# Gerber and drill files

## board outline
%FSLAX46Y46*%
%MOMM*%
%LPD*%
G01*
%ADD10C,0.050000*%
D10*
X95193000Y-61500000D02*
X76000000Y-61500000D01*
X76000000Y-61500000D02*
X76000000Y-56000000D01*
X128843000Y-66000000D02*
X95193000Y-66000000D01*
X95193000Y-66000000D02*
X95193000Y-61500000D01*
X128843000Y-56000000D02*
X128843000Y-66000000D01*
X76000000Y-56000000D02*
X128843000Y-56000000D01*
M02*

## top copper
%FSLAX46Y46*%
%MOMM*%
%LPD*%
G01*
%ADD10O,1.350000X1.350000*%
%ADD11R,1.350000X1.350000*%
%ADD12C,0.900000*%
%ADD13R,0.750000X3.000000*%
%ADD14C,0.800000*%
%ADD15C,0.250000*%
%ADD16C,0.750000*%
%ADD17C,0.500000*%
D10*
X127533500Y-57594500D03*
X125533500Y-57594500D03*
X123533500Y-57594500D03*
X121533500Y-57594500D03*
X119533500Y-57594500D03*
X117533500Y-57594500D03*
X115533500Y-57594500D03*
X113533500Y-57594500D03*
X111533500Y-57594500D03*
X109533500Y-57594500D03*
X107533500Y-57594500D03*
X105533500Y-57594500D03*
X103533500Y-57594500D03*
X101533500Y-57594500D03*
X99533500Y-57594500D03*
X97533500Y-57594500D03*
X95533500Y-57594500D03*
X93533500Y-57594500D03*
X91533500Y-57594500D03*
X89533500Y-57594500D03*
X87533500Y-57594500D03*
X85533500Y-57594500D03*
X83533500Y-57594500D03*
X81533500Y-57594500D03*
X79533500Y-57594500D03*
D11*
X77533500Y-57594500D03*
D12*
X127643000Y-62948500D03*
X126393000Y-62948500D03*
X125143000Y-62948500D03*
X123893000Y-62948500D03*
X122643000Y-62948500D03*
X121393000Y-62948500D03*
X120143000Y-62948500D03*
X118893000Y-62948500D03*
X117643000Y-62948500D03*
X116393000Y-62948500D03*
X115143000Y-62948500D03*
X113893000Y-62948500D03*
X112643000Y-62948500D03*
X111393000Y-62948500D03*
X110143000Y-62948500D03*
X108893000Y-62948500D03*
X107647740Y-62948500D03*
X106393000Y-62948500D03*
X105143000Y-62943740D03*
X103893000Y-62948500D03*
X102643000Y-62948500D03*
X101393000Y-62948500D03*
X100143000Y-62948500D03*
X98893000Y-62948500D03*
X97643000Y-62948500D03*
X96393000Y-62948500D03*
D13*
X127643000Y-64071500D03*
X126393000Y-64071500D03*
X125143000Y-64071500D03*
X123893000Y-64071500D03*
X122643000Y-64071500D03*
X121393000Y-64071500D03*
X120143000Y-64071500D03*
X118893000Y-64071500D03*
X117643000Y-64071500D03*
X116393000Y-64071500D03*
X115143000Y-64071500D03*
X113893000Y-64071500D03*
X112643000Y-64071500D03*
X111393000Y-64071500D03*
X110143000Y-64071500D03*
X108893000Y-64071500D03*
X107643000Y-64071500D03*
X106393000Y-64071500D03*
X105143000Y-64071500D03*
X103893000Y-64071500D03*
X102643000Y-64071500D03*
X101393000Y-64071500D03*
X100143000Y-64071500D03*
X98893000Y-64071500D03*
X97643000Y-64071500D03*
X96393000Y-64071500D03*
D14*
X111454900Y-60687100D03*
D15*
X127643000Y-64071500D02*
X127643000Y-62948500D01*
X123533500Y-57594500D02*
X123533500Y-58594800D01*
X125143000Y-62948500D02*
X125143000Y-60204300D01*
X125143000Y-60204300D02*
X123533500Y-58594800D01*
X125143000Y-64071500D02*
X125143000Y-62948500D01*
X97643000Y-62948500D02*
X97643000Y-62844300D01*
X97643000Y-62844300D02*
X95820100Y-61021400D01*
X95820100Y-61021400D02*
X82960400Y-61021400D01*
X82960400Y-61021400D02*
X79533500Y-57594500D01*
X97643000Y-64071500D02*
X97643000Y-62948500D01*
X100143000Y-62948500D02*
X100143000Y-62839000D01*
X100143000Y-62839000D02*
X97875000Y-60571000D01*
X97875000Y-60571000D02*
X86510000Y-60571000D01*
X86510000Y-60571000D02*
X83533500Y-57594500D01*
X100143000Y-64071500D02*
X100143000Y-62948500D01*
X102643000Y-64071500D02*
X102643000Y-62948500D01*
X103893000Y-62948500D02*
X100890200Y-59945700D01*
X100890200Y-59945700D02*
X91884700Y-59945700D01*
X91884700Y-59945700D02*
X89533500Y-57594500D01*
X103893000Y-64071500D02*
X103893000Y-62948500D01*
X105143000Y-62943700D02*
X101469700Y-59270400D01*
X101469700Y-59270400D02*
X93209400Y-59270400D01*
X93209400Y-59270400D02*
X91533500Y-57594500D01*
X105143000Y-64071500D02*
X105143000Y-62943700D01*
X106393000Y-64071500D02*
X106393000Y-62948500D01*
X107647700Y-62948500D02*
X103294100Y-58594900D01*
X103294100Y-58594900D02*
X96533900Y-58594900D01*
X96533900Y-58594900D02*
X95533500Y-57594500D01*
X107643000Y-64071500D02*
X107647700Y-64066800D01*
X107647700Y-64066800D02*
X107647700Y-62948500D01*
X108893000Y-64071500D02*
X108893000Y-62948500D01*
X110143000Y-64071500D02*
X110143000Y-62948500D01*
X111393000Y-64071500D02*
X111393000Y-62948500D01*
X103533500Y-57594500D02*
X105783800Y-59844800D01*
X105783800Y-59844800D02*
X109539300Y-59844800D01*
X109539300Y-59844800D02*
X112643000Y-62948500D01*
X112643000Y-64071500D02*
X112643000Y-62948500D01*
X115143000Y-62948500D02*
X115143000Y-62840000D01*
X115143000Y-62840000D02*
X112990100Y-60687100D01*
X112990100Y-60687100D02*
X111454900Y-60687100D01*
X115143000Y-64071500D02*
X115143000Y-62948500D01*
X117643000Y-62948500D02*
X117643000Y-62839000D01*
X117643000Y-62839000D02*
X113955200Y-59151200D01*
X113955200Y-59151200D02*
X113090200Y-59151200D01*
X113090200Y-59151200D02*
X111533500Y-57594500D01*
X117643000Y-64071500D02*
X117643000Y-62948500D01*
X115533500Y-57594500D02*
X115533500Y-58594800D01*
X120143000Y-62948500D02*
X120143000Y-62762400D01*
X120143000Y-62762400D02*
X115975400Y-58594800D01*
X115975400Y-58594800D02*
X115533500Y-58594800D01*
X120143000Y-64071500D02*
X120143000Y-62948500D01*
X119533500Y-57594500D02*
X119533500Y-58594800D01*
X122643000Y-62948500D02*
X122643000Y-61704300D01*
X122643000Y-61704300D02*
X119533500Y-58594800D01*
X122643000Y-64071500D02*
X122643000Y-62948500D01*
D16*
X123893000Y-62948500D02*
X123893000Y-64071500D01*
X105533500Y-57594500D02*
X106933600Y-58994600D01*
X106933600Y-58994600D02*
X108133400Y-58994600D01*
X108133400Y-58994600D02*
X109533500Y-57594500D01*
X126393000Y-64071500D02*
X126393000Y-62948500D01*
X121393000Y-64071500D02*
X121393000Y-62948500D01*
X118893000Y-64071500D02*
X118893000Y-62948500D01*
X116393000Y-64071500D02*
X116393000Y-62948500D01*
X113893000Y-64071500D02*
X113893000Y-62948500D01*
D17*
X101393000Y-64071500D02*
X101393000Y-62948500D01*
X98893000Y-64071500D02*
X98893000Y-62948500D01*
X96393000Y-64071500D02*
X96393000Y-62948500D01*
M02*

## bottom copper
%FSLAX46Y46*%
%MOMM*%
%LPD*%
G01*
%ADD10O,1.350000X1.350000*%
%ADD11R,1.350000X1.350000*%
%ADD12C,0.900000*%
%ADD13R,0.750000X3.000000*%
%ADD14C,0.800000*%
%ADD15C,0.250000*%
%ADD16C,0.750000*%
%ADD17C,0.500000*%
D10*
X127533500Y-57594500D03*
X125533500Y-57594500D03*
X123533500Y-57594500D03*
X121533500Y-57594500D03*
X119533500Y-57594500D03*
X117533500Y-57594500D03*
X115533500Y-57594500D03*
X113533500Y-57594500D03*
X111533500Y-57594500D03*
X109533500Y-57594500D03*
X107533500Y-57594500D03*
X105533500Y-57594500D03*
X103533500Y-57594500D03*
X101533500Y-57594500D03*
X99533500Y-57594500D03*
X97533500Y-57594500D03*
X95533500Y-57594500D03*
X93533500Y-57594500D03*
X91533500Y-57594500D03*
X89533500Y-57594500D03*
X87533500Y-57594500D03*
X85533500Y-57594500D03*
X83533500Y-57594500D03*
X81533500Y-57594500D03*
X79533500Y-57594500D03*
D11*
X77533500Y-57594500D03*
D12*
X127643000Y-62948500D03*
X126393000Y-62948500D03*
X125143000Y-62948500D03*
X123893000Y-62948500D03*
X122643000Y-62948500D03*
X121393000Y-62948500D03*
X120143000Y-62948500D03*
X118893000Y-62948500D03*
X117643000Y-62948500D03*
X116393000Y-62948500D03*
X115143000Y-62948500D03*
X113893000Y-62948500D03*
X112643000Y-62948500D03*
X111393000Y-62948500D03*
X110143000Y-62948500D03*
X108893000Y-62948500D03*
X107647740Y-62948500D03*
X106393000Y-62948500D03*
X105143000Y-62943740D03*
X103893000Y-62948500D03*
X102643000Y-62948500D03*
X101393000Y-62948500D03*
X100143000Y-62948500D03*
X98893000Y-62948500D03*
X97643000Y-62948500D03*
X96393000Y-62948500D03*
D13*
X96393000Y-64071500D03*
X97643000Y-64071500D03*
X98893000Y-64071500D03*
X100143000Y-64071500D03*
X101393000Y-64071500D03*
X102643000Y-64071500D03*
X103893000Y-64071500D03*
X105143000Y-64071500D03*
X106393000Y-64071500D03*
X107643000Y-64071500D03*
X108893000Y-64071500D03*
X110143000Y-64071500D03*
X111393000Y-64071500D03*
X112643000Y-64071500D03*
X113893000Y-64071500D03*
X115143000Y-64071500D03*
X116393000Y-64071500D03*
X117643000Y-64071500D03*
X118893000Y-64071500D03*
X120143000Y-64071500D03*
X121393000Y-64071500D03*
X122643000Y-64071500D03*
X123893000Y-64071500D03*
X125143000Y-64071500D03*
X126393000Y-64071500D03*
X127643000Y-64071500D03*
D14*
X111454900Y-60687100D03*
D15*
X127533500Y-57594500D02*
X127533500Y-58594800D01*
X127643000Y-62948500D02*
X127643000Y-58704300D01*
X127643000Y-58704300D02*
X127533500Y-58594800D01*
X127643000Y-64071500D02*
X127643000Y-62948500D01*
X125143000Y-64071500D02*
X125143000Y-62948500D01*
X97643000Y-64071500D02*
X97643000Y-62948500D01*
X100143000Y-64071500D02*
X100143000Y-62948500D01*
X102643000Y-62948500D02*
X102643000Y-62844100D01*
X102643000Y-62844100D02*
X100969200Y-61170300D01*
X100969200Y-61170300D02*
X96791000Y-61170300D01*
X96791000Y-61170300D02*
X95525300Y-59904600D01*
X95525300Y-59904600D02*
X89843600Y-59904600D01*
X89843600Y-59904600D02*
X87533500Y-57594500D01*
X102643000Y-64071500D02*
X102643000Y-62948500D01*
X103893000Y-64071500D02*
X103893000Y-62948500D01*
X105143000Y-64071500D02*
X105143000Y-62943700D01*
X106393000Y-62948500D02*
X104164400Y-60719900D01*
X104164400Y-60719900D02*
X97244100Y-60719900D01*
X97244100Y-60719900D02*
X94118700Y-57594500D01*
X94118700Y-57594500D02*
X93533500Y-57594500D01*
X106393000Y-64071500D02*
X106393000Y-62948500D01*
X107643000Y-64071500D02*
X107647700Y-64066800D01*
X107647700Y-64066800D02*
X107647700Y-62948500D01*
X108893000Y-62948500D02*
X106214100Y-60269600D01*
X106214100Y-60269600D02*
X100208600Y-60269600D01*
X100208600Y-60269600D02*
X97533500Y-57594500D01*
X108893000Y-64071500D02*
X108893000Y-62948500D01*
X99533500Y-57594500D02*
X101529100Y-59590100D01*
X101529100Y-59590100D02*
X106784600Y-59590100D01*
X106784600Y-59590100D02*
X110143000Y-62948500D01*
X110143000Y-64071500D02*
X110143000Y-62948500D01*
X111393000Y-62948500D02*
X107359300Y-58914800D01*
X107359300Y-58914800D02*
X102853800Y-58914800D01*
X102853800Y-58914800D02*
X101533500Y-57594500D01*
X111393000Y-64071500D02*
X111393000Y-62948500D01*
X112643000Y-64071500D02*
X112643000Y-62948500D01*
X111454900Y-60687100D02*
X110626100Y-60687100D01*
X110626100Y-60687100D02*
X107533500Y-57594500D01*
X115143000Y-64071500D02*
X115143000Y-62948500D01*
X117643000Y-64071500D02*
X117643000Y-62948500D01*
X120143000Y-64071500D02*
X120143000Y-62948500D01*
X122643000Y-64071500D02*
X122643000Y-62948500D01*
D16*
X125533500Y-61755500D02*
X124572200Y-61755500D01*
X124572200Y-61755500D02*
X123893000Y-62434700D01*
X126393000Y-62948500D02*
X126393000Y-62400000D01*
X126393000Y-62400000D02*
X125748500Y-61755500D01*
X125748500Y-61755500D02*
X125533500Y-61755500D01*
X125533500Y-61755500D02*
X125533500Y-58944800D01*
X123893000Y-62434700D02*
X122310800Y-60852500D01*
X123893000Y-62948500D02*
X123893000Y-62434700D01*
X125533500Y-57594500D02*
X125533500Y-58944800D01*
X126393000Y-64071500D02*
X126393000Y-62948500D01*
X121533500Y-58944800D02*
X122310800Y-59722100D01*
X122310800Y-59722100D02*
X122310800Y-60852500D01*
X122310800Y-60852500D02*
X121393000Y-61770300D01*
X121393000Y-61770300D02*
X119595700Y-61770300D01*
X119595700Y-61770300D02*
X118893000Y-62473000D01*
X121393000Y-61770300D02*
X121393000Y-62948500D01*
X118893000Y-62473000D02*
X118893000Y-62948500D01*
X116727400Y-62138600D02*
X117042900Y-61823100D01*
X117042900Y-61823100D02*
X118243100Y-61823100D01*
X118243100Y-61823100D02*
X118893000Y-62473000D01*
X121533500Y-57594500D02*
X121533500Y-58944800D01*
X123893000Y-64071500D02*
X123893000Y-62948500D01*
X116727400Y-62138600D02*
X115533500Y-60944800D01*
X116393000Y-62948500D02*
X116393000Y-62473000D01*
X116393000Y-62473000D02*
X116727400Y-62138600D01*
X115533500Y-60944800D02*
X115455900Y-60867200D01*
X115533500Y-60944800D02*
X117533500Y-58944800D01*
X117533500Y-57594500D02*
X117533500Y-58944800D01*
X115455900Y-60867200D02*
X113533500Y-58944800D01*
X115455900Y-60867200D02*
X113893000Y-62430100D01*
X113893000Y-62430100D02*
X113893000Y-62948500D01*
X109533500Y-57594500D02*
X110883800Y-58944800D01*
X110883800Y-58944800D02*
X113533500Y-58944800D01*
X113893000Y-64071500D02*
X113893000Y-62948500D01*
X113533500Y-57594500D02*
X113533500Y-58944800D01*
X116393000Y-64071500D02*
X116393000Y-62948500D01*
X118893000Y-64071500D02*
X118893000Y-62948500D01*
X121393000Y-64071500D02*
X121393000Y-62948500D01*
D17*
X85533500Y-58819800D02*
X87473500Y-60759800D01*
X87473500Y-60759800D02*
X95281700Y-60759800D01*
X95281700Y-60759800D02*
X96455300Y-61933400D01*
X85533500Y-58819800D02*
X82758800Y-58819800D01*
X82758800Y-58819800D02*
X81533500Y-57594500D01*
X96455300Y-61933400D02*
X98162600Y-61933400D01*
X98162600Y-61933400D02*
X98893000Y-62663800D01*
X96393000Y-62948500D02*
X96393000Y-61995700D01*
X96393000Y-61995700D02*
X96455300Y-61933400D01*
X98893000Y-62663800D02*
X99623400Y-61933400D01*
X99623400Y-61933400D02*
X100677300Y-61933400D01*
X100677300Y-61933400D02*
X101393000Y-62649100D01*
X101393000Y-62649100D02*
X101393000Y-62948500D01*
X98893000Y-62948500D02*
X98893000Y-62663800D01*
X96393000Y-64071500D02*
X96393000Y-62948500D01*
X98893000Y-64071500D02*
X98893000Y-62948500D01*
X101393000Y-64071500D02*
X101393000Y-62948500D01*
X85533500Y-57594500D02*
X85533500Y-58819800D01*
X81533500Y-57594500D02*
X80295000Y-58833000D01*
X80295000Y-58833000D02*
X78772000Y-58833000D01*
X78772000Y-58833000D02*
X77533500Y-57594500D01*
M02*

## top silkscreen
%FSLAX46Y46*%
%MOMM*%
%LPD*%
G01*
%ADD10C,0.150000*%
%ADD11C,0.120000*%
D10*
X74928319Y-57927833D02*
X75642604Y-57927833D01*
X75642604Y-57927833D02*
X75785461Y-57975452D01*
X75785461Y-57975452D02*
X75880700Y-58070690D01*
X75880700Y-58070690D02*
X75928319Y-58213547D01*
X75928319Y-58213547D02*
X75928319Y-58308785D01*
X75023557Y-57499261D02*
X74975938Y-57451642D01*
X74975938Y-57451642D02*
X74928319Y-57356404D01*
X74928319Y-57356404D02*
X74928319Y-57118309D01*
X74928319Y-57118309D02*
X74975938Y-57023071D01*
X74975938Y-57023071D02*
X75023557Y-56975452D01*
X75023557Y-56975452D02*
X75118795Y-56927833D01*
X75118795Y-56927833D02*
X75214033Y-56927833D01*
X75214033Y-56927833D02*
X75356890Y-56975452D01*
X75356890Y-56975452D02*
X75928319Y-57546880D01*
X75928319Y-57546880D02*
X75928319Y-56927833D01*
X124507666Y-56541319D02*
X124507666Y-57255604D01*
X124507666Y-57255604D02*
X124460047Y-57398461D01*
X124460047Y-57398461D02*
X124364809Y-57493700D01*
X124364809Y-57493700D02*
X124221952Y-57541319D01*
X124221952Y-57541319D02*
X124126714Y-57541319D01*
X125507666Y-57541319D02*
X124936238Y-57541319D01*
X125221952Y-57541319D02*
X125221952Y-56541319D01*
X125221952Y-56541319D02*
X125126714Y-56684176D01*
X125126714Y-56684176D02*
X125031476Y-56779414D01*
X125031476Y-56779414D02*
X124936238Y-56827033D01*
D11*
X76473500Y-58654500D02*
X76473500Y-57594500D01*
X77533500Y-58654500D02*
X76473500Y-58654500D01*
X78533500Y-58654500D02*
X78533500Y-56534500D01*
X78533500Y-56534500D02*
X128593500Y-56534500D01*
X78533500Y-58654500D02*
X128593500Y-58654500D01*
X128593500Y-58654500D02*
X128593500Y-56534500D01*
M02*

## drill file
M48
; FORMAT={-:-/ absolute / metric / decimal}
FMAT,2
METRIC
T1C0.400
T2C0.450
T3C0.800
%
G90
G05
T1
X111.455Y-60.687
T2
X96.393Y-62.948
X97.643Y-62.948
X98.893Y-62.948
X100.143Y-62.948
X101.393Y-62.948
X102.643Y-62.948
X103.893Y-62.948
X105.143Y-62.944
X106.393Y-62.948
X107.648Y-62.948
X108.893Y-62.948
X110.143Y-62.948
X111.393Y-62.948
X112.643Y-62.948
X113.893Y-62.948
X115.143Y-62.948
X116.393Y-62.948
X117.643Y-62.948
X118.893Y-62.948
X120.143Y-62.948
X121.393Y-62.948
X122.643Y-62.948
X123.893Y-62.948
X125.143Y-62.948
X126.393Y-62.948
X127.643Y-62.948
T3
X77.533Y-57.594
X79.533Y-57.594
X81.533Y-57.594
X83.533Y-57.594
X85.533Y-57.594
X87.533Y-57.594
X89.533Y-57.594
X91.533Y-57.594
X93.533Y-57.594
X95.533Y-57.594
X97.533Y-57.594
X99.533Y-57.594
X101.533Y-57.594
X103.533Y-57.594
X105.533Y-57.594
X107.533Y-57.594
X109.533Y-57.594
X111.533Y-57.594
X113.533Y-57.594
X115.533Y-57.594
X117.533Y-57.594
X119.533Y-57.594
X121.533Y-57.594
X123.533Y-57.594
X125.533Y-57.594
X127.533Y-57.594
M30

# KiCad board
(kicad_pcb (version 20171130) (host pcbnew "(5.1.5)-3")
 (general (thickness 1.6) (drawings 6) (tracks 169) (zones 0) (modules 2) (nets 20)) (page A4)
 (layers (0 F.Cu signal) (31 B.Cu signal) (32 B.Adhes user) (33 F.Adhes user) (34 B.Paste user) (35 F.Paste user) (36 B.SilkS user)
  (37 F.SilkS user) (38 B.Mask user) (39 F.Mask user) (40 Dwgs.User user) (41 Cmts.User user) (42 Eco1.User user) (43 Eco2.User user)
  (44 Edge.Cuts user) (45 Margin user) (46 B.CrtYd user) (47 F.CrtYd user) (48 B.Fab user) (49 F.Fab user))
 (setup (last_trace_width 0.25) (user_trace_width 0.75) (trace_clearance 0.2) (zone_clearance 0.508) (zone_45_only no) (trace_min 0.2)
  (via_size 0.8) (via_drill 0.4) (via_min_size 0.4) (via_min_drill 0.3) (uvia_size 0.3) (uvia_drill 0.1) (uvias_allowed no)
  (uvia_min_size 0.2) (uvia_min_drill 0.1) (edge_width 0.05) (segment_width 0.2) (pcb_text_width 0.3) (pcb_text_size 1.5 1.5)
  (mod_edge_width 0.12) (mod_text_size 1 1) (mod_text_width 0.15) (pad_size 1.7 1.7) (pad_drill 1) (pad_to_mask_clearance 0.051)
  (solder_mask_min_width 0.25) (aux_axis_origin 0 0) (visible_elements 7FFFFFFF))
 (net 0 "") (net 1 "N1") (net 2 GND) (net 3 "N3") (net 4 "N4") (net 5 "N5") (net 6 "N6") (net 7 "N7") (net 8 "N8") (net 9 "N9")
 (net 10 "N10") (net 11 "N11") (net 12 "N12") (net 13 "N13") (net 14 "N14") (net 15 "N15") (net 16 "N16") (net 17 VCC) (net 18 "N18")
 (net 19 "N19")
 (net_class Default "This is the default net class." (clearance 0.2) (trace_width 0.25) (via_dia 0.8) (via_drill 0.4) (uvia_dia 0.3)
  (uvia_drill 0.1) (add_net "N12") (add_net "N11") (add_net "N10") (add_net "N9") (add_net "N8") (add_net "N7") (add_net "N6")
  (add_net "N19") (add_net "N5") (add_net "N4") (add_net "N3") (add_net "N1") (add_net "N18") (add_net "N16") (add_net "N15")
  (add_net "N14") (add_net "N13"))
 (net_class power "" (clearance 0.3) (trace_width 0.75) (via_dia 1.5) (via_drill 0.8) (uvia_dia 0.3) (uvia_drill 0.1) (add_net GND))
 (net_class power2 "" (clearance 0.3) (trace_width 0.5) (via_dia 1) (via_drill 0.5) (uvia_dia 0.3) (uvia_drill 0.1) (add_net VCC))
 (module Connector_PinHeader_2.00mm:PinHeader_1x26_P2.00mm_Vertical (layer F.Cu) (at 77.5335 57.5945 90)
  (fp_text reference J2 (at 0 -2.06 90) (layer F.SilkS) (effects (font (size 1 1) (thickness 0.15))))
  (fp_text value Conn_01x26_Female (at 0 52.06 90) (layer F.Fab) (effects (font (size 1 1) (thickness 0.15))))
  (fp_line (start -1.06 -1.06) (end 0 -1.06) (layer F.SilkS) (width 0.12))
  (fp_line (start -1.06 0) (end -1.06 -1.06) (layer F.SilkS) (width 0.12))
  (fp_line (start -1.06 1) (end 1.06 1) (layer F.SilkS) (width 0.12))
  (fp_line (start 1.06 1) (end 1.06 51.06) (layer F.SilkS) (width 0.12))
  (fp_line (start -1.06 1) (end -1.06 51.06) (layer F.SilkS) (width 0.12))
  (fp_line (start -1.06 51.06) (end 1.06 51.06) (layer F.SilkS) (width 0.12))
  (pad 26 thru_hole oval (at 0 50 90) (size 1.35 1.35) (drill 0.8) (layers *.Cu *.Mask) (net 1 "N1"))
  (pad 25 thru_hole oval (at 0 48 90) (size 1.35 1.35) (drill 0.8) (layers *.Cu *.Mask) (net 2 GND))
  (pad 24 thru_hole oval (at 0 46 90) (size 1.35 1.35) (drill 0.8) (layers *.Cu *.Mask) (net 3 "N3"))
  (pad 23 thru_hole oval (at 0 44 90) (size 1.35 1.35) (drill 0.8) (layers *.Cu *.Mask) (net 2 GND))
  (pad 22 thru_hole oval (at 0 42 90) (size 1.35 1.35) (drill 0.8) (layers *.Cu *.Mask) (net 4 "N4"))
  (pad 21 thru_hole oval (at 0 40 90) (size 1.35 1.35) (drill 0.8) (layers *.Cu *.Mask) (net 2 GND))
  (pad 20 thru_hole oval (at 0 38 90) (size 1.35 1.35) (drill 0.8) (layers *.Cu *.Mask) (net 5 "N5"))
  (pad 19 thru_hole oval (at 0 36 90) (size 1.35 1.35) (drill 0.8) (layers *.Cu *.Mask) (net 2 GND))
  (pad 18 thru_hole oval (at 0 34 90) (size 1.35 1.35) (drill 0.8) (layers *.Cu *.Mask) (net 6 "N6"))
  (pad 17 thru_hole oval (at 0 32 90) (size 1.35 1.35) (drill 0.8) (layers *.Cu *.Mask) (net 2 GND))
  (pad 16 thru_hole oval (at 0 30 90) (size 1.35 1.35) (drill 0.8) (layers *.Cu *.Mask) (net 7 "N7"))
  (pad 15 thru_hole oval (at 0 28 90) (size 1.35 1.35) (drill 0.8) (layers *.Cu *.Mask) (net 2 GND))
  (pad 14 thru_hole oval (at 0 26 90) (size 1.35 1.35) (drill 0.8) (layers *.Cu *.Mask) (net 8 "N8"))
  (pad 13 thru_hole oval (at 0 24 90) (size 1.35 1.35) (drill 0.8) (layers *.Cu *.Mask) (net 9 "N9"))
  (pad 12 thru_hole oval (at 0 22 90) (size 1.35 1.35) (drill 0.8) (layers *.Cu *.Mask) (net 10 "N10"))
  (pad 11 thru_hole oval (at 0 20 90) (size 1.35 1.35) (drill 0.8) (layers *.Cu *.Mask) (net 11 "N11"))
  (pad 10 thru_hole oval (at 0 18 90) (size 1.35 1.35) (drill 0.8) (layers *.Cu *.Mask) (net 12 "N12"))
  (pad 9 thru_hole oval (at 0 16 90) (size 1.35 1.35) (drill 0.8) (layers *.Cu *.Mask) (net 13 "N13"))
  (pad 8 thru_hole oval (at 0 14 90) (size 1.35 1.35) (drill 0.8) (layers *.Cu *.Mask) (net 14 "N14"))
  (pad 7 thru_hole oval (at 0 12 90) (size 1.35 1.35) (drill 0.8) (layers *.Cu *.Mask) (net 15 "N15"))
  (pad 6 thru_hole oval (at 0 10 90) (size 1.35 1.35) (drill 0.8) (layers *.Cu *.Mask) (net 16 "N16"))
  (pad 5 thru_hole oval (at 0 8 90) (size 1.35 1.35) (drill 0.8) (layers *.Cu *.Mask) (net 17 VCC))
  (pad 4 thru_hole oval (at 0 6 90) (size 1.35 1.35) (drill 0.8) (layers *.Cu *.Mask) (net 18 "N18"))
  (pad 3 thru_hole oval (at 0 4 90) (size 1.35 1.35) (drill 0.8) (layers *.Cu *.Mask) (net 17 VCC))
  (pad 2 thru_hole oval (at 0 2 90) (size 1.35 1.35) (drill 0.8) (layers *.Cu *.Mask) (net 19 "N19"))
  (pad 1 thru_hole rect (at 0 0 90) (size 1.35 1.35) (drill 0.8) (layers *.Cu *.Mask) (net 17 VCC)))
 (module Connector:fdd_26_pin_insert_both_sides (layer F.Cu) (at 96.393 64.1985)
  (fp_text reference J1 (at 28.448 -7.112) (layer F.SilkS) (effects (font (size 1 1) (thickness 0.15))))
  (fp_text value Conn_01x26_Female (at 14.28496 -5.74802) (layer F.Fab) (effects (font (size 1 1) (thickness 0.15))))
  (pad 26 thru_hole circle (at 31.25 -1.25) (size 0.9 0.9) (drill 0.45) (layers *.Cu *.Mask) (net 1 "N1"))
  (pad 25 thru_hole circle (at 30 -1.25) (size 0.9 0.9) (drill 0.45) (layers *.Cu *.Mask) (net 2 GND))
  (pad 24 thru_hole circle (at 28.75 -1.25) (size 0.9 0.9) (drill 0.45) (layers *.Cu *.Mask) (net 3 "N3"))
  (pad 23 thru_hole circle (at 27.5 -1.25) (size 0.9 0.9) (drill 0.45) (layers *.Cu *.Mask) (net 2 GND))
  (pad 22 thru_hole circle (at 26.25 -1.25) (size 0.9 0.9) (drill 0.45) (layers *.Cu *.Mask) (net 4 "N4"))
  (pad 21 thru_hole circle (at 25 -1.25) (size 0.9 0.9) (drill 0.45) (layers *.Cu *.Mask) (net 2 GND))
  (pad 20 thru_hole circle (at 23.75 -1.25) (size 0.9 0.9) (drill 0.45) (layers *.Cu *.Mask) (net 5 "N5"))
  (pad 19 thru_hole circle (at 22.5 -1.25) (size 0.9 0.9) (drill 0.45) (layers *.Cu *.Mask) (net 2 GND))
  (pad 18 thru_hole circle (at 21.25 -1.25) (size 0.9 0.9) (drill 0.45) (layers *.Cu *.Mask) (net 6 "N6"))
  (pad 17 thru_hole circle (at 20 -1.25) (size 0.9 0.9) (drill 0.45) (layers *.Cu *.Mask) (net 2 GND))
  (pad 16 thru_hole circle (at 18.75 -1.25) (size 0.9 0.9) (drill 0.45) (layers *.Cu *.Mask) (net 7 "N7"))
  (pad 15 thru_hole circle (at 17.5 -1.25 90) (size 0.9 0.9) (drill 0.45) (layers *.Cu *.Mask) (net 2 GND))
  (pad 14 thru_hole circle (at 16.25 -1.25) (size 0.9 0.9) (drill 0.45) (layers *.Cu *.Mask) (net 8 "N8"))
  (pad 13 thru_hole circle (at 15 -1.25) (size 0.9 0.9) (drill 0.45) (layers *.Cu *.Mask) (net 9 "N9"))
  (pad 12 thru_hole circle (at 13.75 -1.25) (size 0.9 0.9) (drill 0.45) (layers *.Cu *.Mask) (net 10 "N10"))
  (pad 11 thru_hole circle (at 12.5 -1.25) (size 0.9 0.9) (drill 0.45) (layers *.Cu *.Mask) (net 11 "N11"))
  (pad 10 thru_hole circle (at 11.25474 -1.25) (size 0.9 0.9) (drill 0.45) (layers *.Cu *.Mask) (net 12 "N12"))
  (pad 9 thru_hole circle (at 10 -1.25) (size 0.9 0.9) (drill 0.45) (layers *.Cu *.Mask) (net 13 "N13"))
  (pad 8 thru_hole circle (at 8.75 -1.25476) (size 0.9 0.9) (drill 0.45) (layers *.Cu *.Mask) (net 14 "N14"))
  (pad 7 thru_hole circle (at 7.5 -1.25) (size 0.9 0.9) (drill 0.45) (layers *.Cu *.Mask) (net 15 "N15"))
  (pad 6 thru_hole circle (at 6.25 -1.25) (size 0.9 0.9) (drill 0.45) (layers *.Cu *.Mask) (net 16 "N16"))
  (pad 5 thru_hole circle (at 5 -1.25) (size 0.9 0.9) (drill 0.45) (layers *.Cu *.Mask) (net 17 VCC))
  (pad 4 thru_hole circle (at 3.75 -1.25) (size 0.9 0.9) (drill 0.45) (layers *.Cu *.Mask) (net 18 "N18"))
  (pad 3 thru_hole circle (at 2.5 -1.25) (size 0.9 0.9) (drill 0.45) (layers *.Cu *.Mask) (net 17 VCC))
  (pad 2 thru_hole circle (at 1.25 -1.25 90) (size 0.9 0.9) (drill 0.45) (layers *.Cu *.Mask) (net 19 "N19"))
  (pad 1 thru_hole circle (at 0 -1.25) (size 0.9 0.9) (drill 0.45) (layers *.Cu *.Mask) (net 17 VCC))
  (pad 26 connect rect (at 31.25 -0.127) (size 0.75 3) (layers F.Cu B.Mask) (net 1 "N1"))
  (pad 25 connect rect (at 30 -0.127) (size 0.75 3) (layers F.Cu B.Mask) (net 2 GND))
  (pad 24 connect rect (at 28.75 -0.127) (size 0.75 3) (layers F.Cu B.Mask) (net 3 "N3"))
  (pad 23 connect rect (at 27.5 -0.127) (size 0.75 3) (layers F.Cu B.Mask) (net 2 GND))
  (pad 22 connect rect (at 26.25 -0.127) (size 0.75 3) (layers F.Cu B.Mask) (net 4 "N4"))
  (pad 21 connect rect (at 25 -0.127) (size 0.75 3) (layers F.Cu B.Mask) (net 2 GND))
  (pad 20 connect rect (at 23.75 -0.127) (size 0.75 3) (layers F.Cu B.Mask) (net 5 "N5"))
  (pad 19 connect rect (at 22.5 -0.127) (size 0.75 3) (layers F.Cu B.Mask) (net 2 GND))
  (pad 18 connect rect (at 21.25 -0.127) (size 0.75 3) (layers F.Cu B.Mask) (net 6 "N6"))
  (pad 17 connect rect (at 20 -0.127) (size 0.75 3) (layers F.Cu B.Mask) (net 2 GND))
  (pad 16 connect rect (at 18.75 -0.127) (size 0.75 3) (layers F.Cu B.Mask) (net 7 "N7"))
  (pad 15 connect rect (at 17.5 -0.127) (size 0.75 3) (layers F.Cu B.Mask) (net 2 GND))
  (pad 14 connect rect (at 16.25 -0.127) (size 0.75 3) (layers F.Cu B.Mask) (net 8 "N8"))
  (pad 13 connect rect (at 15 -0.127) (size 0.75 3) (layers F.Cu B.Mask) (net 9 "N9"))
  (pad 12 connect rect (at 13.75 -0.127) (size 0.75 3) (layers F.Cu B.Mask) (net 10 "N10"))
  (pad 11 connect rect (at 12.5 -0.127) (size 0.75 3) (layers F.Cu B.Mask) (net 11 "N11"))
  (pad 10 connect rect (at 11.25 -0.127) (size 0.75 3) (layers F.Cu B.Mask) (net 12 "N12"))
  (pad 9 connect rect (at 10 -0.127) (size 0.75 3) (layers F.Cu B.Mask) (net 13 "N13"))
  (pad 8 connect rect (at 8.75 -0.127) (size 0.75 3) (layers F.Cu B.Mask) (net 14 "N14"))
  (pad 7 connect rect (at 7.5 -0.127) (size 0.75 3) (layers F.Cu B.Mask) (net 15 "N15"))
  (pad 6 connect rect (at 6.25 -0.127) (size 0.75 3) (layers F.Cu B.Mask) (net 16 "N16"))
  (pad 5 connect rect (at 5 -0.127) (size 0.75 3) (layers F.Cu B.Mask) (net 17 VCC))
  (pad 4 connect rect (at 3.75 -0.127) (size 0.75 3) (layers F.Cu B.Mask) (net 18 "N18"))
  (pad 3 connect rect (at 2.5 -0.127) (size 0.75 3) (layers F.Cu B.Mask) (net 17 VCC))
  (pad 2 connect rect (at 1.25 -0.127) (size 0.75 3) (layers F.Cu B.Mask) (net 19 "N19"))
  (pad 1 connect rect (at 0 -0.127) (size 0.75 3) (layers F.Cu B.Mask) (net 17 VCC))
  (pad 1 connect rect (at 0 -0.127) (size 0.75 3) (layers B.Cu B.Mask) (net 17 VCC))
  (pad 2 connect rect (at 1.25 -0.127) (size 0.75 3) (layers B.Cu B.Mask) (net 19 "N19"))
  (pad 3 connect rect (at 2.5 -0.127) (size 0.75 3) (layers B.Cu B.Mask) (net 17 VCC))
  (pad 4 connect rect (at 3.75 -0.127) (size 0.75 3) (layers B.Cu B.Mask) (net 18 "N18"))
  (pad 5 connect rect (at 5 -0.127) (size 0.75 3) (layers B.Cu B.Mask) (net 17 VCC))
  (pad 6 connect rect (at 6.25 -0.127) (size 0.75 3) (layers B.Cu B.Mask) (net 16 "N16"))
  (pad 7 connect rect (at 7.5 -0.127) (size 0.75 3) (layers B.Cu B.Mask) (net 15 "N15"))
  (pad 8 connect rect (at 8.75 -0.127) (size 0.75 3) (layers B.Cu B.Mask) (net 14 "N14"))
  (pad 9 connect rect (at 10 -0.127) (size 0.75 3) (layers B.Cu B.Mask) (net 13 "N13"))
  (pad 10 connect rect (at 11.25 -0.127) (size 0.75 3) (layers B.Cu B.Mask) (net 12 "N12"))
  (pad 11 connect rect (at 12.5 -0.127) (size 0.75 3) (layers B.Cu B.Mask) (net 11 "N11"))
  (pad 12 connect rect (at 13.75 -0.127) (size 0.75 3) (layers B.Cu B.Mask) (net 10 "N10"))
  (pad 13 connect rect (at 15 -0.127) (size 0.75 3) (layers B.Cu B.Mask) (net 9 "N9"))
  (pad 14 connect rect (at 16.25 -0.127) (size 0.75 3) (layers B.Cu B.Mask) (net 8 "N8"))
  (pad 15 connect rect (at 17.5 -0.127) (size 0.75 3) (layers B.Cu B.Mask) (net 2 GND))
  (pad 16 connect rect (at 18.75 -0.127) (size 0.75 3) (layers B.Cu B.Mask) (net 7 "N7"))
  (pad 17 connect rect (at 20 -0.127) (size 0.75 3) (layers B.Cu B.Mask) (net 2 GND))
  (pad 18 connect rect (at 21.25 -0.127) (size 0.75 3) (layers B.Cu B.Mask) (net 6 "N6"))
  (pad 19 connect rect (at 22.5 -0.127) (size 0.75 3) (layers B.Cu B.Mask) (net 2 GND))
  (pad 20 connect rect (at 23.75 -0.127) (size 0.75 3) (layers B.Cu B.Mask) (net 5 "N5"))
  (pad 21 connect rect (at 25 -0.127) (size 0.75 3) (layers B.Cu B.Mask) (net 2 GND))
  (pad 22 connect rect (at 26.25 -0.127) (size 0.75 3) (layers B.Cu B.Mask) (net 4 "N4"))
  (pad 23 connect rect (at 27.5 -0.127) (size 0.75 3) (layers B.Cu B.Mask) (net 2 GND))
  (pad 24 connect rect (at 28.75 -0.127) (size 0.75 3) (layers B.Cu B.Mask) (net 3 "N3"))
  (pad 25 connect rect (at 30 -0.127) (size 0.75 3) (layers B.Cu B.Mask) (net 2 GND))
  (pad 26 connect rect (at 31.25 -0.127) (size 0.75 3) (layers B.Cu B.Mask) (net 1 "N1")))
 (gr_line (start 95.193 61.5) (end 76 61.5) (layer Edge.Cuts) (width 0.05))
 (gr_line (start 76 61.5) (end 76 56) (layer Edge.Cuts) (width 0.05))
 (gr_line (start 128.843 66) (end 95.193 66) (layer Edge.Cuts) (width 0.05))
 (gr_line (start 95.193 66) (end 95.193 61.5) (layer Edge.Cuts) (width 0.05))
 (gr_line (start 128.843 56) (end 128.843 66) (layer Edge.Cuts) (width 0.05))
 (gr_line (start 76 56) (end 128.843 56) (layer Edge.Cuts) (width 0.05))
 (segment (start 127.5335 57.5945) (end 127.5335 58.5948) (width 0.25) (layer B.Cu) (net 1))
 (segment (start 127.643 62.9485) (end 127.643 58.7043) (width 0.25) (layer B.Cu) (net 1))
 (segment (start 127.643 58.7043) (end 127.5335 58.5948) (width 0.25) (layer B.Cu) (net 1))
 (segment (start 127.643 64.0715) (end 127.643 62.9485) (width 0.25) (layer B.Cu) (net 1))
 (segment (start 127.643 64.0715) (end 127.643 62.9485) (width 0.25) (layer F.Cu) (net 1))
 (segment (start 123.5335 57.5945) (end 123.5335 58.5948) (width 0.25) (layer F.Cu) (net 3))
 (segment (start 125.143 62.9485) (end 125.143 60.2043) (width 0.25) (layer F.Cu) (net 3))
 (segment (start 125.143 60.2043) (end 123.5335 58.5948) (width 0.25) (layer F.Cu) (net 3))
 (segment (start 125.143 64.0715) (end 125.143 62.9485) (width 0.25) (layer F.Cu) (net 3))
 (segment (start 125.143 64.0715) (end 125.143 62.9485) (width 0.25) (layer B.Cu) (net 3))
 (segment (start 97.643 62.9485) (end 97.643 62.8443) (width 0.25) (layer F.Cu) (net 19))
 (segment (start 97.643 62.8443) (end 95.8201 61.0214) (width 0.25) (layer F.Cu) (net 19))
 (segment (start 95.8201 61.0214) (end 82.9604 61.0214) (width 0.25) (layer F.Cu) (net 19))
 (segment (start 82.9604 61.0214) (end 79.5335 57.5945) (width 0.25) (layer F.Cu) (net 19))
 (segment (start 97.643 64.0715) (end 97.643 62.9485) (width 0.25) (layer F.Cu) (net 19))
 (segment (start 97.643 64.0715) (end 97.643 62.9485) (width 0.25) (layer B.Cu) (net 19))
 (segment (start 100.143 62.9485) (end 100.143 62.839) (width 0.25) (layer F.Cu) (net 18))
 (segment (start 100.143 62.839) (end 97.875 60.571) (width 0.25) (layer F.Cu) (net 18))
 (segment (start 97.875 60.571) (end 86.51 60.571) (width 0.25) (layer F.Cu) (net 18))
 (segment (start 86.51 60.571) (end 83.5335 57.5945) (width 0.25) (layer F.Cu) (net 18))
 (segment (start 100.143 64.0715) (end 100.143 62.9485) (width 0.25) (layer F.Cu) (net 18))
 (segment (start 100.143 64.0715) (end 100.143 62.9485) (width 0.25) (layer B.Cu) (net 18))
 (segment (start 102.643 62.9485) (end 102.643 62.8441) (width 0.25) (layer B.Cu) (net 16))
 (segment (start 102.643 62.8441) (end 100.9692 61.1703) (width 0.25) (layer B.Cu) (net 16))
 (segment (start 100.9692 61.1703) (end 96.791 61.1703) (width 0.25) (layer B.Cu) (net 16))
 (segment (start 96.791 61.1703) (end 95.5253 59.9046) (width 0.25) (layer B.Cu) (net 16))
 (segment (start 95.5253 59.9046) (end 89.8436 59.9046) (width 0.25) (layer B.Cu) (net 16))
 (segment (start 89.8436 59.9046) (end 87.5335 57.5945) (width 0.25) (layer B.Cu) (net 16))
 (segment (start 102.643 64.0715) (end 102.643 62.9485) (width 0.25) (layer B.Cu) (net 16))
 (segment (start 102.643 64.0715) (end 102.643 62.9485) (width 0.25) (layer F.Cu) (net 16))
 (segment (start 103.893 62.9485) (end 100.8902 59.9457) (width 0.25) (layer F.Cu) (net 15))
 (segment (start 100.8902 59.9457) (end 91.8847 59.9457) (width 0.25) (layer F.Cu) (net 15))
 (segment (start 91.8847 59.9457) (end 89.5335 57.5945) (width 0.25) (layer F.Cu) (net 15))
 (segment (start 103.893 64.0715) (end 103.893 62.9485) (width 0.25) (layer F.Cu) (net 15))
 (segment (start 103.893 64.0715) (end 103.893 62.9485) (width 0.25) (layer B.Cu) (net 15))
 (segment (start 105.143 62.9437) (end 101.4697 59.2704) (width 0.25) (layer F.Cu) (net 14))
 (segment (start 101.4697 59.2704) (end 93.2094 59.2704) (width 0.25) (layer F.Cu) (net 14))
 (segment (start 93.2094 59.2704) (end 91.5335 57.5945) (width 0.25) (layer F.Cu) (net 14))
 (segment (start 105.143 64.0715) (end 105.143 62.9437) (width 0.25) (layer F.Cu) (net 14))
 (segment (start 105.143 64.0715) (end 105.143 62.9437) (width 0.25) (layer B.Cu) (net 14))
 (segment (start 106.393 62.9485) (end 104.1644 60.7199) (width 0.25) (layer B.Cu) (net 13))
 (segment (start 104.1644 60.7199) (end 97.2441 60.7199) (width 0.25) (layer B.Cu) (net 13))
 (segment (start 97.2441 60.7199) (end 94.1187 57.5945) (width 0.25) (layer B.Cu) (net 13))
 (segment (start 94.1187 57.5945) (end 93.5335 57.5945) (width 0.25) (layer B.Cu) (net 13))
 (segment (start 106.393 64.0715) (end 106.393 62.9485) (width 0.25) (layer B.Cu) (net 13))
 (segment (start 106.393 64.0715) (end 106.393 62.9485) (width 0.25) (layer F.Cu) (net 13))
 (segment (start 107.6477 62.9485) (end 103.2941 58.5949) (width 0.25) (layer F.Cu) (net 12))
 (segment (start 103.2941 58.5949) (end 96.5339 58.5949) (width 0.25) (layer F.Cu) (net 12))
 (segment (start 96.5339 58.5949) (end 95.5335 57.5945) (width 0.25) (layer F.Cu) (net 12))
 (segment (start 107.643 64.0715) (end 107.6477 64.0668) (width 0.25) (layer F.Cu) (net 12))
 (segment (start 107.6477 64.0668) (end 107.6477 62.9485) (width 0.25) (layer F.Cu) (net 12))
 (segment (start 107.643 64.0715) (end 107.6477 64.0668) (width 0.25) (layer B.Cu) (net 12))
 (segment (start 107.6477 64.0668) (end 107.6477 62.9485) (width 0.25) (layer B.Cu) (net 12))
 (segment (start 108.893 62.9485) (end 106.2141 60.2696) (width 0.25) (layer B.Cu) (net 11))
 (segment (start 106.2141 60.2696) (end 100.2086 60.2696) (width 0.25) (layer B.Cu) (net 11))
 (segment (start 100.2086 60.2696) (end 97.5335 57.5945) (width 0.25) (layer B.Cu) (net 11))
 (segment (start 108.893 64.0715) (end 108.893 62.9485) (width 0.25) (layer B.Cu) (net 11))
 (segment (start 108.893 64.0715) (end 108.893 62.9485) (width 0.25) (layer F.Cu) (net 11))
 (segment (start 99.5335 57.5945) (end 101.5291 59.5901) (width 0.25) (layer B.Cu) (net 10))
 (segment (start 101.5291 59.5901) (end 106.7846 59.5901) (width 0.25) (layer B.Cu) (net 10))
 (segment (start 106.7846 59.5901) (end 110.143 62.9485) (width 0.25) (layer B.Cu) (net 10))
 (segment (start 110.143 64.0715) (end 110.143 62.9485) (width 0.25) (layer B.Cu) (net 10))
 (segment (start 110.143 64.0715) (end 110.143 62.9485) (width 0.25) (layer F.Cu) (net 10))
 (segment (start 111.393 62.9485) (end 107.3593 58.9148) (width 0.25) (layer B.Cu) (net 9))
 (segment (start 107.3593 58.9148) (end 102.8538 58.9148) (width 0.25) (layer B.Cu) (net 9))
 (segment (start 102.8538 58.9148) (end 101.5335 57.5945) (width 0.25) (layer B.Cu) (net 9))
 (segment (start 111.393 64.0715) (end 111.393 62.9485) (width 0.25) (layer B.Cu) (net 9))
 (segment (start 111.393 64.0715) (end 111.393 62.9485) (width 0.25) (layer F.Cu) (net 9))
 (segment (start 103.5335 57.5945) (end 105.7838 59.8448) (width 0.25) (layer F.Cu) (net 8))
 (segment (start 105.7838 59.8448) (end 109.5393 59.8448) (width 0.25) (layer F.Cu) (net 8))
 (segment (start 109.5393 59.8448) (end 112.643 62.9485) (width 0.25) (layer F.Cu) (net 8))
 (segment (start 112.643 64.0715) (end 112.643 62.9485) (width 0.25) (layer F.Cu) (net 8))
 (segment (start 112.643 64.0715) (end 112.643 62.9485) (width 0.25) (layer B.Cu) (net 8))
 (segment (start 115.143 62.9485) (end 115.143 62.84) (width 0.25) (layer F.Cu) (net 7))
 (segment (start 115.143 62.84) (end 112.9901 60.6871) (width 0.25) (layer F.Cu) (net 7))
 (segment (start 112.9901 60.6871) (end 111.4549 60.6871) (width 0.25) (layer F.Cu) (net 7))
 (segment (start 111.4549 60.6871) (end 110.6261 60.6871) (width 0.25) (layer B.Cu) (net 7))
 (segment (start 110.6261 60.6871) (end 107.5335 57.5945) (width 0.25) (layer B.Cu) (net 7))
 (segment (start 115.143 64.0715) (end 115.143 62.9485) (width 0.25) (layer F.Cu) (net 7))
 (segment (start 115.143 64.0715) (end 115.143 62.9485) (width 0.25) (layer B.Cu) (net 7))
 (via (at 111.4549 60.6871) (size 0.8) (layers F.Cu B.Cu) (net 7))
 (segment (start 117.643 62.9485) (end 117.643 62.839) (width 0.25) (layer F.Cu) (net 6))
 (segment (start 117.643 62.839) (end 113.9552 59.1512) (width 0.25) (layer F.Cu) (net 6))
 (segment (start 113.9552 59.1512) (end 113.0902 59.1512) (width 0.25) (layer F.Cu) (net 6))
 (segment (start 113.0902 59.1512) (end 111.5335 57.5945) (width 0.25) (layer F.Cu) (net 6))
 (segment (start 117.643 64.0715) (end 117.643 62.9485) (width 0.25) (layer F.Cu) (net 6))
 (segment (start 117.643 64.0715) (end 117.643 62.9485) (width 0.25) (layer B.Cu) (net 6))
 (segment (start 115.5335 57.5945) (end 115.5335 58.5948) (width 0.25) (layer F.Cu) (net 5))
 (segment (start 120.143 62.9485) (end 120.143 62.7624) (width 0.25) (layer F.Cu) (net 5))
 (segment (start 120.143 62.7624) (end 115.9754 58.5948) (width 0.25) (layer F.Cu) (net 5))
 (segment (start 115.9754 58.5948) (end 115.5335 58.5948) (width 0.25) (layer F.Cu) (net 5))
 (segment (start 120.143 64.0715) (end 120.143 62.9485) (width 0.25) (layer F.Cu) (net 5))
 (segment (start 120.143 64.0715) (end 120.143 62.9485) (width 0.25) (layer B.Cu) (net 5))
 (segment (start 119.5335 57.5945) (end 119.5335 58.5948) (width 0.25) (layer F.Cu) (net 4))
 (segment (start 122.643 62.9485) (end 122.643 61.7043) (width 0.25) (layer F.Cu) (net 4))
 (segment (start 122.643 61.7043) (end 119.5335 58.5948) (width 0.25) (layer F.Cu) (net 4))
 (segment (start 122.643 64.0715) (end 122.643 62.9485) (width 0.25) (layer F.Cu) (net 4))
 (segment (start 122.643 64.0715) (end 122.643 62.9485) (width 0.25) (layer B.Cu) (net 4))
 (segment (start 125.5335 61.7555) (end 124.5722 61.7555) (width 0.75) (layer B.Cu) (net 2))
 (segment (start 124.5722 61.7555) (end 123.893 62.4347) (width 0.75) (layer B.Cu) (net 2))
 (segment (start 126.393 62.9485) (end 126.393 62.4) (width 0.75) (layer B.Cu) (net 2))
 (segment (start 126.393 62.4) (end 125.7485 61.7555) (width 0.75) (layer B.Cu) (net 2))
 (segment (start 125.7485 61.7555) (end 125.5335 61.7555) (width 0.75) (layer B.Cu) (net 2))
 (segment (start 125.5335 61.7555) (end 125.5335 58.9448) (width 0.75) (layer B.Cu) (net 2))
 (segment (start 123.893 62.4347) (end 122.3108 60.8525) (width 0.75) (layer B.Cu) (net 2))
 (segment (start 123.893 62.9485) (end 123.893 62.4347) (width 0.75) (layer B.Cu) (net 2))
 (segment (start 125.5335 57.5945) (end 125.5335 58.9448) (width 0.75) (layer B.Cu) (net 2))
 (segment (start 126.393 64.0715) (end 126.393 62.9485) (width 0.75) (layer B.Cu) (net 2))
 (segment (start 123.893 62.9485) (end 123.893 64.0715) (width 0.75) (layer F.Cu) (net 2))
 (segment (start 121.5335 58.9448) (end 122.3108 59.7221) (width 0.75) (layer B.Cu) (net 2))
 (segment (start 122.3108 59.7221) (end 122.3108 60.8525) (width 0.75) (layer B.Cu) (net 2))
 (segment (start 122.3108 60.8525) (end 121.393 61.7703) (width 0.75) (layer B.Cu) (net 2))
 (segment (start 121.393 61.7703) (end 119.5957 61.7703) (width 0.75) (layer B.Cu) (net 2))
 (segment (start 119.5957 61.7703) (end 118.893 62.473) (width 0.75) (layer B.Cu) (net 2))
 (segment (start 121.393 61.7703) (end 121.393 62.9485) (width 0.75) (layer B.Cu) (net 2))
 (segment (start 118.893 62.473) (end 118.893 62.9485) (width 0.75) (layer B.Cu) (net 2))
 (segment (start 116.7274 62.1386) (end 117.0429 61.8231) (width 0.75) (layer B.Cu) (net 2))
 (segment (start 117.0429 61.8231) (end 118.2431 61.8231) (width 0.75) (layer B.Cu) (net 2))
 (segment (start 118.2431 61.8231) (end 118.893 62.473) (width 0.75) (layer B.Cu) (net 2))
 (segment (start 121.5335 57.5945) (end 121.5335 58.9448) (width 0.75) (layer B.Cu) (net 2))
 (segment (start 123.893 64.0715) (end 123.893 62.9485) (width 0.75) (layer B.Cu) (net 2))
 (segment (start 116.7274 62.1386) (end 115.5335 60.9448) (width 0.75) (layer B.Cu) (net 2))
 (segment (start 116.393 62.9485) (end 116.393 62.473) (width 0.75) (layer B.Cu) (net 2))
 (segment (start 116.393 62.473) (end 116.7274 62.1386) (width 0.75) (layer B.Cu) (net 2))
 (segment (start 115.5335 60.9448) (end 115.4559 60.8672) (width 0.75) (layer B.Cu) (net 2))
 (segment (start 115.5335 60.9448) (end 117.5335 58.9448) (width 0.75) (layer B.Cu) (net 2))
 (segment (start 117.5335 57.5945) (end 117.5335 58.9448) (width 0.75) (layer B.Cu) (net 2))
 (segment (start 115.4559 60.8672) (end 113.5335 58.9448) (width 0.75) (layer B.Cu) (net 2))
 (segment (start 115.4559 60.8672) (end 113.893 62.4301) (width 0.75) (layer B.Cu) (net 2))
 (segment (start 113.893 62.4301) (end 113.893 62.9485) (width 0.75) (layer B.Cu) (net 2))
 (segment (start 109.5335 57.5945) (end 110.8838 58.9448) (width 0.75) (layer B.Cu) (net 2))
 (segment (start 110.8838 58.9448) (end 113.5335 58.9448) (width 0.75) (layer B.Cu) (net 2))
 (segment (start 113.893 64.0715) (end 113.893 62.9485) (width 0.75) (layer B.Cu) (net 2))
 (segment (start 113.5335 57.5945) (end 113.5335 58.9448) (width 0.75) (layer B.Cu) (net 2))
 (segment (start 105.5335 57.5945) (end 106.9336 58.9946) (width 0.75) (layer F.Cu) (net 2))
 (segment (start 106.9336 58.9946) (end 108.1334 58.9946) (width 0.75) (layer F.Cu) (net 2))
 (segment (start 108.1334 58.9946) (end 109.5335 57.5945) (width 0.75) (layer F.Cu) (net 2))
 (segment (start 126.393 64.0715) (end 126.393 62.9485) (width 0.75) (layer F.Cu) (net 2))
 (segment (start 121.393 64.0715) (end 121.393 62.9485) (width 0.75) (layer F.Cu) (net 2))
 (segment (start 118.893 64.0715) (end 118.893 62.9485) (width 0.75) (layer F.Cu) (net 2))
 (segment (start 116.393 64.0715) (end 116.393 62.9485) (width 0.75) (layer F.Cu) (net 2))
 (segment (start 113.893 64.0715) (end 113.893 62.9485) (width 0.75) (layer F.Cu) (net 2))
 (segment (start 116.393 64.0715) (end 116.393 62.9485) (width 0.75) (layer B.Cu) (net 2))
 (segment (start 118.893 64.0715) (end 118.893 62.9485) (width 0.75) (layer B.Cu) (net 2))
 (segment (start 121.393 64.0715) (end 121.393 62.9485) (width 0.75) (layer B.Cu) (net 2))
 (segment (start 85.5335 58.8198) (end 87.4735 60.7598) (width 0.5) (layer B.Cu) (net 17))
 (segment (start 87.4735 60.7598) (end 95.2817 60.7598) (width 0.5) (layer B.Cu) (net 17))
 (segment (start 95.2817 60.7598) (end 96.4553 61.9334) (width 0.5) (layer B.Cu) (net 17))
 (segment (start 85.5335 58.8198) (end 82.7588 58.8198) (width 0.5) (layer B.Cu) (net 17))
 (segment (start 82.7588 58.8198) (end 81.5335 57.5945) (width 0.5) (layer B.Cu) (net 17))
 (segment (start 96.4553 61.9334) (end 98.1626 61.9334) (width 0.5) (layer B.Cu) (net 17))
 (segment (start 98.1626 61.9334) (end 98.893 62.6638) (width 0.5) (layer B.Cu) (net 17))
 (segment (start 96.393 62.9485) (end 96.393 61.9957) (width 0.5) (layer B.Cu) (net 17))
 (segment (start 96.393 61.9957) (end 96.4553 61.9334) (width 0.5) (layer B.Cu) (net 17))
 (segment (start 98.893 62.6638) (end 99.6234 61.9334) (width 0.5) (layer B.Cu) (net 17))
 (segment (start 99.6234 61.9334) (end 100.6773 61.9334) (width 0.5) (layer B.Cu) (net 17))
 (segment (start 100.6773 61.9334) (end 101.393 62.6491) (width 0.5) (layer B.Cu) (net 17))
 (segment (start 101.393 62.6491) (end 101.393 62.9485) (width 0.5) (layer B.Cu) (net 17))
 (segment (start 98.893 62.9485) (end 98.893 62.6638) (width 0.5) (layer B.Cu) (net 17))
 (segment (start 96.393 64.0715) (end 96.393 62.9485) (width 0.5) (layer B.Cu) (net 17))
 (segment (start 98.893 64.0715) (end 98.893 62.9485) (width 0.5) (layer B.Cu) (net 17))
 (segment (start 101.393 64.0715) (end 101.393 62.9485) (width 0.5) (layer B.Cu) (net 17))
 (segment (start 85.5335 57.5945) (end 85.5335 58.8198) (width 0.5) (layer B.Cu) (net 17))
 (segment (start 81.5335 57.5945) (end 80.295 58.833) (width 0.5) (layer B.Cu) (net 17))
 (segment (start 80.295 58.833) (end 78.772 58.833) (width 0.5) (layer B.Cu) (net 17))
 (segment (start 78.772 58.833) (end 77.5335 57.5945) (width 0.5) (layer B.Cu) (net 17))
 (segment (start 101.393 64.0715) (end 101.393 62.9485) (width 0.5) (layer F.Cu) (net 17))
 (segment (start 98.893 64.0715) (end 98.893 62.9485) (width 0.5) (layer F.Cu) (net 17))
 (segment (start 96.393 64.0715) (end 96.393 62.9485) (width 0.5) (layer F.Cu) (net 17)))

